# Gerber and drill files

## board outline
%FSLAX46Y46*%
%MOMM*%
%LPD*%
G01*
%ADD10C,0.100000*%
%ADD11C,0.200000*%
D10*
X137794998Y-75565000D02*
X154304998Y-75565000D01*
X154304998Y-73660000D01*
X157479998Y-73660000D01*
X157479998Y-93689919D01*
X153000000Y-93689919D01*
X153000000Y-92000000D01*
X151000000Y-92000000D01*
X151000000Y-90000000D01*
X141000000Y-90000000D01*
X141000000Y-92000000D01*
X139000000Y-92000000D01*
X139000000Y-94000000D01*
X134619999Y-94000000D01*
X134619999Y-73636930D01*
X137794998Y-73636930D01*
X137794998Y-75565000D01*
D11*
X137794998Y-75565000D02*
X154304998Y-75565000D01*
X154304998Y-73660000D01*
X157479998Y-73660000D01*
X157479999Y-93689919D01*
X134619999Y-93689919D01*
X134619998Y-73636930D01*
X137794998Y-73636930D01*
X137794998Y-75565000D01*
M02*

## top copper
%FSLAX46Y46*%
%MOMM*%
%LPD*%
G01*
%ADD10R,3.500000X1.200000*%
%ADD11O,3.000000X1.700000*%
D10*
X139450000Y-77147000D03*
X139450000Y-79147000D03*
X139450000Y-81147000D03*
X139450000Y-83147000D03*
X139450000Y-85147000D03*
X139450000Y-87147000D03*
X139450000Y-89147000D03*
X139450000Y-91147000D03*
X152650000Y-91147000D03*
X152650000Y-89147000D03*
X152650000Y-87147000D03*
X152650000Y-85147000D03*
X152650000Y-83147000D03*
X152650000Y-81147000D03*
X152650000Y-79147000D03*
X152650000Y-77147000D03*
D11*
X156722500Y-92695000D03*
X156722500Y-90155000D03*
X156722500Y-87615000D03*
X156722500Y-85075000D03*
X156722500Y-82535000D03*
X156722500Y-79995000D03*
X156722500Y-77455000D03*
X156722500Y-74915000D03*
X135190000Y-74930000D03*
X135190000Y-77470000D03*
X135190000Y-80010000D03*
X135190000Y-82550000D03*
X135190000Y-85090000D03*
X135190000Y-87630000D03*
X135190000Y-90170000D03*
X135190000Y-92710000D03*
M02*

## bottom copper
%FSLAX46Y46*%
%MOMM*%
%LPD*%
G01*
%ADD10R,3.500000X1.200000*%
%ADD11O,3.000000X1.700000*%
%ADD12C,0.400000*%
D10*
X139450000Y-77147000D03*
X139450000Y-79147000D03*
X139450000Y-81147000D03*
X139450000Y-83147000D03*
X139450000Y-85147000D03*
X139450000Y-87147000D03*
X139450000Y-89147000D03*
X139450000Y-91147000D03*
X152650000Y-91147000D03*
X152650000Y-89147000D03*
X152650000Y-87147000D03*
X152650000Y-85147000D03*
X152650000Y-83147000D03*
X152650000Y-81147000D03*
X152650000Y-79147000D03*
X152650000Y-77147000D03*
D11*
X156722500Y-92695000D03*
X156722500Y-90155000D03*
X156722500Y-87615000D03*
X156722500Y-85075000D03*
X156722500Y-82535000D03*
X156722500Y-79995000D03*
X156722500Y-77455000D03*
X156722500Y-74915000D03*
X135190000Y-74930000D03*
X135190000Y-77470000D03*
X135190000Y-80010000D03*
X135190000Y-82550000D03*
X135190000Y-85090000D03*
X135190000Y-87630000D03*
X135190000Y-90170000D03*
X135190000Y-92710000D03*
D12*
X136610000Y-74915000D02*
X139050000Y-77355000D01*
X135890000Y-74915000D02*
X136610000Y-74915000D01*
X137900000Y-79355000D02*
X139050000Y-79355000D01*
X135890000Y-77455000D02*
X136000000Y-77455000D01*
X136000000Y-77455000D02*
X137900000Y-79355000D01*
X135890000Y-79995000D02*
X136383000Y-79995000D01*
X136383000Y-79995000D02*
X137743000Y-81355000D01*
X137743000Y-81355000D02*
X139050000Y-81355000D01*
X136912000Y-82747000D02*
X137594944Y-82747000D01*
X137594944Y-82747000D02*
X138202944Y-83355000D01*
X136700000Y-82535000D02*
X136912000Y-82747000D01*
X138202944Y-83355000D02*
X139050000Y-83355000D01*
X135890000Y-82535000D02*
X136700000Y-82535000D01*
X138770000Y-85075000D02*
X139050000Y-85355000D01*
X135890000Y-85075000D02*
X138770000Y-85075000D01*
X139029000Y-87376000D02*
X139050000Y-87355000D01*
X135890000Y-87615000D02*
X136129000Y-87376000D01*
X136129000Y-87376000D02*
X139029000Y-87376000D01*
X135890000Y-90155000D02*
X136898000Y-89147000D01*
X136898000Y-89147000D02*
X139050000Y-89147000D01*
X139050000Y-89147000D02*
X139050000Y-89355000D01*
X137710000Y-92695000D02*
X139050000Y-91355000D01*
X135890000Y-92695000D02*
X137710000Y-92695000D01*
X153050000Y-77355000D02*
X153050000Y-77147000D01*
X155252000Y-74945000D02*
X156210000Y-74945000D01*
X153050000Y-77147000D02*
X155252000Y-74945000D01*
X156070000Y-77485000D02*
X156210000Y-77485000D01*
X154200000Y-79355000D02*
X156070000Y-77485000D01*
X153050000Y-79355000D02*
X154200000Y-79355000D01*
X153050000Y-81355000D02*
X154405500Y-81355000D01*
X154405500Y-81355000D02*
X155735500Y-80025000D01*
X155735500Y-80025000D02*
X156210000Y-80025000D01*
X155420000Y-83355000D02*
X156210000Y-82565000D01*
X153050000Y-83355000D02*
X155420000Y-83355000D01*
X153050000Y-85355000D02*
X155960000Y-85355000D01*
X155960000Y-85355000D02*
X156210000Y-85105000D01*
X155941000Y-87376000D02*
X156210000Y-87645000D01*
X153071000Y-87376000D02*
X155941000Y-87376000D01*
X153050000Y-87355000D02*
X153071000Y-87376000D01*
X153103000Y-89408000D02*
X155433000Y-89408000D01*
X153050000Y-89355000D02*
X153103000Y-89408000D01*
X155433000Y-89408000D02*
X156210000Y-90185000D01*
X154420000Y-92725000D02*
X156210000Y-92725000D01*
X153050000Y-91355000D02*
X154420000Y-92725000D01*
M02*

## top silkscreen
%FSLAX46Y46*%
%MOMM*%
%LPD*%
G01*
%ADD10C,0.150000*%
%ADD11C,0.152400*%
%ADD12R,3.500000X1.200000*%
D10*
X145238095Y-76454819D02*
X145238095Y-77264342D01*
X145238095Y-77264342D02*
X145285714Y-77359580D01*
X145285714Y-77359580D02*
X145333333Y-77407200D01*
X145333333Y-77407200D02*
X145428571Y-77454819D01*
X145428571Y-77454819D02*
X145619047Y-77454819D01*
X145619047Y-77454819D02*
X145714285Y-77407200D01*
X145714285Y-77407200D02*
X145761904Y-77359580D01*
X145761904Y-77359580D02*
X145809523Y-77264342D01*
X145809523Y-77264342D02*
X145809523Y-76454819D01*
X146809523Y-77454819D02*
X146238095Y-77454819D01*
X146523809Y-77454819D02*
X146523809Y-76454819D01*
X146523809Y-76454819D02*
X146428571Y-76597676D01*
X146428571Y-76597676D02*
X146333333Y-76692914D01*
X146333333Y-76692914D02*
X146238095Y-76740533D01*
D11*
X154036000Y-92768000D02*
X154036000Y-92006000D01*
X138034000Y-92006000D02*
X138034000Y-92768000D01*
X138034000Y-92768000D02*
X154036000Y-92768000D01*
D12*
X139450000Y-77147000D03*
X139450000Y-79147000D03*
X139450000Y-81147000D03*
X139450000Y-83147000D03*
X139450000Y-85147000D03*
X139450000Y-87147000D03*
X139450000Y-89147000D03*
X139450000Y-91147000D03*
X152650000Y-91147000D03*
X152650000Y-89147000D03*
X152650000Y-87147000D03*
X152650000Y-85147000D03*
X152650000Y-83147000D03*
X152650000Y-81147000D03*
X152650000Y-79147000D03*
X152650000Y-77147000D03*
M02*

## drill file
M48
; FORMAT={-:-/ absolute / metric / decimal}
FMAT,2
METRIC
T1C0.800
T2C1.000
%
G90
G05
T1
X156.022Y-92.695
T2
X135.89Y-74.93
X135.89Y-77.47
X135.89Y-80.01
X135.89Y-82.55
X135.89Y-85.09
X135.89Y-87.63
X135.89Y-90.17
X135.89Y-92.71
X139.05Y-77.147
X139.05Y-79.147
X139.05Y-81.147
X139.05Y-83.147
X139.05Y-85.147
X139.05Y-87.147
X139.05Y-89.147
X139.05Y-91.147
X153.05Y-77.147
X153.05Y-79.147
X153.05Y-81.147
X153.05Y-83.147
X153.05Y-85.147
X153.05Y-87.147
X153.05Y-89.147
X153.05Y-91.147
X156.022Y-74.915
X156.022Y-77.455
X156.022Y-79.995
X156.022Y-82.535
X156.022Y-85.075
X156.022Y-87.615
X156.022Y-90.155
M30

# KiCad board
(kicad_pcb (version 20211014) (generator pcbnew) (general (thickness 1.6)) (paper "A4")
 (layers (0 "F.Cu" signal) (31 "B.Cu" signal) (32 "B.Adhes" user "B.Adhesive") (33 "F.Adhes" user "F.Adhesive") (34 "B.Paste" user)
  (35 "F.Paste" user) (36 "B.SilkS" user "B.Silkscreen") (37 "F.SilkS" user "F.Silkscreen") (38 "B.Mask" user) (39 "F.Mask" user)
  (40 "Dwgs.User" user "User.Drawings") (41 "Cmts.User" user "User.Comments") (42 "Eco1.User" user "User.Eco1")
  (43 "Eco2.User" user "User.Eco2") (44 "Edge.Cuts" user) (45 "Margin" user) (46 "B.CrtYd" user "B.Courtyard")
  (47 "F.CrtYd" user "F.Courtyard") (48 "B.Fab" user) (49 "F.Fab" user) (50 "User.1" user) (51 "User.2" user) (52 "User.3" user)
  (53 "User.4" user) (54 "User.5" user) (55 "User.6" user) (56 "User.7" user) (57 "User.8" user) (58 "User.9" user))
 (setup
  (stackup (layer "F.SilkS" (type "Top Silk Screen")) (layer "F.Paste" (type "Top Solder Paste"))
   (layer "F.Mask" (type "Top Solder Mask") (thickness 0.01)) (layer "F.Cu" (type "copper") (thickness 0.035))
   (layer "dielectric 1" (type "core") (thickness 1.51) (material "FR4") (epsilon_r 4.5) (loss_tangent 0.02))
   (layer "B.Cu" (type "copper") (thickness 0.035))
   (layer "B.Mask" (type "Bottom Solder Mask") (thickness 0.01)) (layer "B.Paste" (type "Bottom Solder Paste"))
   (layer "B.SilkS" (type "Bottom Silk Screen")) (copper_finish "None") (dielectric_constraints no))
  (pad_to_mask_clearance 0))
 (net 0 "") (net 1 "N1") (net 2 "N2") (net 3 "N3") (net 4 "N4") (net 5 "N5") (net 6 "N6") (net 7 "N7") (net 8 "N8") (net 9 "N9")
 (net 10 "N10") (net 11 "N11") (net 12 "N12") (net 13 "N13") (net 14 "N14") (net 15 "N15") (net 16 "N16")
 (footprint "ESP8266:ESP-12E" (layer "F.Cu") (at 139.05 77.147)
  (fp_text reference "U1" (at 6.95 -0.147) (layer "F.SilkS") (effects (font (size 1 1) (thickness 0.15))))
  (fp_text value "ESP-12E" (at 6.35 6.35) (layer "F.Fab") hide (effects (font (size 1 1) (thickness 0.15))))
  (fp_line (start 14.986 15.621) (end 14.986 14.859) (layer "F.SilkS") (width 0.1524))
  (fp_line (start -1.016 14.859) (end -1.016 15.621) (layer "F.SilkS") (width 0.1524))
  (fp_line (start -1.016 15.621) (end 14.986 15.621) (layer "F.SilkS") (width 0.1524))
  (pad "1" thru_hole rect (at 0 0) (size 3.5 1.2) (drill 1 (offset 0.4 0)) (layers *.Cu *.Mask "F.SilkS") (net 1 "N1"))
  (pad "2" thru_hole rect (at 0 2) (size 3.5 1.2) (drill 1 (offset 0.4 0)) (layers *.Cu *.Mask "F.SilkS") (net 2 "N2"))
  (pad "3" thru_hole rect (at 0 4) (size 3.5 1.2) (drill 1 (offset 0.4 0)) (layers *.Cu *.Mask "F.SilkS") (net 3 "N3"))
  (pad "4" thru_hole rect (at 0 6) (size 3.5 1.2) (drill 1 (offset 0.4 0)) (layers *.Cu *.Mask "F.SilkS") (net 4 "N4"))
  (pad "5" thru_hole rect (at 0 8) (size 3.5 1.2) (drill 1 (offset 0.4 0)) (layers *.Cu *.Mask "F.SilkS") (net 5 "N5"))
  (pad "6" thru_hole rect (at 0 10) (size 3.5 1.2) (drill 1 (offset 0.4 0)) (layers *.Cu *.Mask "F.SilkS") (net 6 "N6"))
  (pad "7" thru_hole rect (at 0 12) (size 3.5 1.2) (drill 1 (offset 0.4 0)) (layers *.Cu *.Mask "F.SilkS") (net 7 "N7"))
  (pad "8" thru_hole rect (at 0 14) (size 3.5 1.2) (drill 1 (offset 0.4 0)) (layers *.Cu *.Mask "F.SilkS") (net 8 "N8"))
  (pad "9" thru_hole rect (at 14 14 180) (size 3.5 1.2) (drill 1 (offset 0.4 0)) (layers *.Cu *.Mask "F.SilkS") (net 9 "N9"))
  (pad "10" thru_hole rect (at 14 12 180) (size 3.5 1.2) (drill 1 (offset 0.4 0)) (layers *.Cu *.Mask "F.SilkS") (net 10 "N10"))
  (pad "11" thru_hole rect (at 14 10 180) (size 3.5 1.2) (drill 1 (offset 0.4 0)) (layers *.Cu *.Mask "F.SilkS") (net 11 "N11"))
  (pad "12" thru_hole rect (at 14 8 180) (size 3.5 1.2) (drill 1 (offset 0.4 0)) (layers *.Cu *.Mask "F.SilkS") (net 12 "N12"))
  (pad "13" thru_hole rect (at 14 6 180) (size 3.5 1.2) (drill 1 (offset 0.4 0)) (layers *.Cu *.Mask "F.SilkS") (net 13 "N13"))
  (pad "14" thru_hole rect (at 14 4 180) (size 3.5 1.2) (drill 1 (offset 0.4 0)) (layers *.Cu *.Mask "F.SilkS") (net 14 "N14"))
  (pad "15" thru_hole rect (at 14 2 180) (size 3.5 1.2) (drill 1 (offset 0.4 0)) (layers *.Cu *.Mask "F.SilkS") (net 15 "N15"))
  (pad "16" thru_hole rect (at 14 0 180) (size 3.5 1.2) (drill 1 (offset 0.4 0)) (layers *.Cu *.Mask "F.SilkS") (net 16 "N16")))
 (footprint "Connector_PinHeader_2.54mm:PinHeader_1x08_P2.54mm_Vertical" (layer "B.Cu") (at 156.0225 92.695)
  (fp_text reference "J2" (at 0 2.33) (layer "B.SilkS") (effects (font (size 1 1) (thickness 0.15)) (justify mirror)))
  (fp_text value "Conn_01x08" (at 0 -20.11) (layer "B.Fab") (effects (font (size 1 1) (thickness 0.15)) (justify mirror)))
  (pad "1" thru_hole oval (at 0 0) (size 3 1.7) (drill 0.8 (offset 0.7 0)) (layers *.Cu *.Mask) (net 9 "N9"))
  (pad "2" thru_hole oval (at 0 -2.54) (size 3 1.7) (drill 1 (offset 0.7 0)) (layers *.Cu *.Mask) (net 10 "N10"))
  (pad "3" thru_hole oval (at 0 -5.08) (size 3 1.7) (drill 1 (offset 0.7 0)) (layers *.Cu *.Mask) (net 11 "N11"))
  (pad "4" thru_hole oval (at 0 -7.62) (size 3 1.7) (drill 1 (offset 0.7 0)) (layers *.Cu *.Mask) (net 12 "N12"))
  (pad "5" thru_hole oval (at 0 -10.16) (size 3 1.7) (drill 1 (offset 0.7 0)) (layers *.Cu *.Mask) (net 13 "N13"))
  (pad "6" thru_hole oval (at 0 -12.7) (size 3 1.7) (drill 1 (offset 0.7 0)) (layers *.Cu *.Mask) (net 14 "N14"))
  (pad "7" thru_hole oval (at 0 -15.24) (size 3 1.7) (drill 1 (offset 0.7 0)) (layers *.Cu *.Mask) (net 15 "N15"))
  (pad "8" thru_hole oval (at 0 -17.78) (size 3 1.7) (drill 1 (offset 0.7 0)) (layers *.Cu *.Mask) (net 16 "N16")))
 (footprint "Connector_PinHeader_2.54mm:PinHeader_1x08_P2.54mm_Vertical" (layer "B.Cu") (at 135.89 74.93 180)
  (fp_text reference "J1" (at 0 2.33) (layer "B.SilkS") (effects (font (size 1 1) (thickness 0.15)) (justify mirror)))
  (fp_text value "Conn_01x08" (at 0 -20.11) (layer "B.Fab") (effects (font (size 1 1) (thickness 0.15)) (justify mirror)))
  (pad "1" thru_hole oval (at 0 0 180) (size 3 1.7) (drill 1 (offset 0.7 0)) (layers *.Cu *.Mask) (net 1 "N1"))
  (pad "2" thru_hole oval (at 0 -2.54 180) (size 3 1.7) (drill 1 (offset 0.7 0)) (layers *.Cu *.Mask) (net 2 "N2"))
  (pad "3" thru_hole oval (at 0 -5.08 180) (size 3 1.7) (drill 1 (offset 0.7 0)) (layers *.Cu *.Mask) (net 3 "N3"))
  (pad "4" thru_hole oval (at 0 -7.62 180) (size 3 1.7) (drill 1 (offset 0.7 0)) (layers *.Cu *.Mask) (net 4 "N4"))
  (pad "5" thru_hole oval (at 0 -10.16 180) (size 3 1.7) (drill 1 (offset 0.7 0)) (layers *.Cu *.Mask) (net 5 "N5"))
  (pad "6" thru_hole oval (at 0 -12.7 180) (size 3 1.7) (drill 1 (offset 0.7 0)) (layers *.Cu *.Mask) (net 6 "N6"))
  (pad "7" thru_hole oval (at 0 -15.24 180) (size 3 1.7) (drill 1 (offset 0.7 0)) (layers *.Cu *.Mask) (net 7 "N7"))
  (pad "8" thru_hole oval (at 0 -17.78 180) (size 3 1.7) (drill 1 (offset 0.7 0)) (layers *.Cu *.Mask) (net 8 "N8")))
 (gr_poly
  (pts (xy 137.794998 75.565) (xy 154.304998 75.565) (xy 154.304998 73.66) (xy 157.479998 73.66) (xy 157.479998 93.689919)
   (xy 153 93.689919) (xy 153 92) (xy 151 92) (xy 151 90) (xy 141 90) (xy 141 92) (xy 139 92) (xy 139 94) (xy 134.619999 94)
   (xy 134.619999 73.63693) (xy 137.794998 73.63693))
  (layer "Edge.Cuts") (width 0.1) (fill none))
 (gr_poly
  (pts (xy 137.794998 75.565) (xy 154.304998 75.565) (xy 154.304998 73.66) (xy 157.479998 73.66) (xy 157.479999 93.689919)
   (xy 134.619999 93.689919) (xy 134.619998 73.63693) (xy 137.794998 73.63693))
  (layer "Edge.Cuts") (width 0.2) (fill none))
 (segment (start 136.61 74.915) (end 139.05 77.355) (width 0.4) (layer "B.Cu") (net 1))
 (segment (start 135.89 74.915) (end 136.61 74.915) (width 0.4) (layer "B.Cu") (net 1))
 (segment (start 137.9 79.355) (end 139.05 79.355) (width 0.4) (layer "B.Cu") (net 2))
 (segment (start 135.89 77.455) (end 136 77.455) (width 0.4) (layer "B.Cu") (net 2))
 (segment (start 136 77.455) (end 137.9 79.355) (width 0.4) (layer "B.Cu") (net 2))
 (segment (start 135.89 79.995) (end 136.383 79.995) (width 0.4) (layer "B.Cu") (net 3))
 (segment (start 136.383 79.995) (end 137.743 81.355) (width 0.4) (layer "B.Cu") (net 3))
 (segment (start 137.743 81.355) (end 139.05 81.355) (width 0.4) (layer "B.Cu") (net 3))
 (segment (start 136.912 82.747) (end 137.594944 82.747) (width 0.4) (layer "B.Cu") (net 4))
 (segment (start 137.594944 82.747) (end 138.202944 83.355) (width 0.4) (layer "B.Cu") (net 4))
 (segment (start 136.7 82.535) (end 136.912 82.747) (width 0.4) (layer "B.Cu") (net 4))
 (segment (start 138.202944 83.355) (end 139.05 83.355) (width 0.4) (layer "B.Cu") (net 4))
 (segment (start 135.89 82.535) (end 136.7 82.535) (width 0.4) (layer "B.Cu") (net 4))
 (segment (start 138.77 85.075) (end 139.05 85.355) (width 0.4) (layer "B.Cu") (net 5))
 (segment (start 135.89 85.075) (end 138.77 85.075) (width 0.4) (layer "B.Cu") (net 5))
 (segment (start 139.029 87.376) (end 139.05 87.355) (width 0.4) (layer "B.Cu") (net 6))
 (segment (start 135.89 87.615) (end 136.129 87.376) (width 0.4) (layer "B.Cu") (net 6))
 (segment (start 136.129 87.376) (end 139.029 87.376) (width 0.4) (layer "B.Cu") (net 6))
 (segment (start 135.89 90.155) (end 136.898 89.147) (width 0.4) (layer "B.Cu") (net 7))
 (segment (start 136.898 89.147) (end 139.05 89.147) (width 0.4) (layer "B.Cu") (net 7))
 (segment (start 139.05 89.147) (end 139.05 89.355) (width 0.4) (layer "B.Cu") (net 7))
 (segment (start 137.71 92.695) (end 139.05 91.355) (width 0.4) (layer "B.Cu") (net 8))
 (segment (start 135.89 92.695) (end 137.71 92.695) (width 0.4) (layer "B.Cu") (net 8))
 (segment (start 153.05 77.355) (end 153.05 77.147) (width 0.4) (layer "B.Cu") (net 16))
 (segment (start 155.252 74.945) (end 156.21 74.945) (width 0.4) (layer "B.Cu") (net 16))
 (segment (start 153.05 77.147) (end 155.252 74.945) (width 0.4) (layer "B.Cu") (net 16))
 (segment (start 156.07 77.485) (end 156.21 77.485) (width 0.4) (layer "B.Cu") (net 15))
 (segment (start 154.2 79.355) (end 156.07 77.485) (width 0.4) (layer "B.Cu") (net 15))
 (segment (start 153.05 79.355) (end 154.2 79.355) (width 0.4) (layer "B.Cu") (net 15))
 (segment (start 153.05 81.355) (end 154.4055 81.355) (width 0.4) (layer "B.Cu") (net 14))
 (segment (start 154.4055 81.355) (end 155.7355 80.025) (width 0.4) (layer "B.Cu") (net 14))
 (segment (start 155.7355 80.025) (end 156.21 80.025) (width 0.4) (layer "B.Cu") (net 14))
 (segment (start 155.42 83.355) (end 156.21 82.565) (width 0.4) (layer "B.Cu") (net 13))
 (segment (start 153.05 83.355) (end 155.42 83.355) (width 0.4) (layer "B.Cu") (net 13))
 (segment (start 153.05 85.355) (end 155.96 85.355) (width 0.4) (layer "B.Cu") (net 12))
 (segment (start 155.96 85.355) (end 156.21 85.105) (width 0.4) (layer "B.Cu") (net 12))
 (segment (start 155.941 87.376) (end 156.21 87.645) (width 0.4) (layer "B.Cu") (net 11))
 (segment (start 153.071 87.376) (end 155.941 87.376) (width 0.4) (layer "B.Cu") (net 11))
 (segment (start 153.05 87.355) (end 153.071 87.376) (width 0.4) (layer "B.Cu") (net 11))
 (segment (start 153.103 89.408) (end 155.433 89.408) (width 0.4) (layer "B.Cu") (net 10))
 (segment (start 153.05 89.355) (end 153.103 89.408) (width 0.4) (layer "B.Cu") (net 10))
 (segment (start 155.433 89.408) (end 156.21 90.185) (width 0.4) (layer "B.Cu") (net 10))
 (segment (start 154.42 92.725) (end 156.21 92.725) (width 0.4) (layer "B.Cu") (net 9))
 (segment (start 153.05 91.355) (end 154.42 92.725) (width 0.4) (layer "B.Cu") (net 9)))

